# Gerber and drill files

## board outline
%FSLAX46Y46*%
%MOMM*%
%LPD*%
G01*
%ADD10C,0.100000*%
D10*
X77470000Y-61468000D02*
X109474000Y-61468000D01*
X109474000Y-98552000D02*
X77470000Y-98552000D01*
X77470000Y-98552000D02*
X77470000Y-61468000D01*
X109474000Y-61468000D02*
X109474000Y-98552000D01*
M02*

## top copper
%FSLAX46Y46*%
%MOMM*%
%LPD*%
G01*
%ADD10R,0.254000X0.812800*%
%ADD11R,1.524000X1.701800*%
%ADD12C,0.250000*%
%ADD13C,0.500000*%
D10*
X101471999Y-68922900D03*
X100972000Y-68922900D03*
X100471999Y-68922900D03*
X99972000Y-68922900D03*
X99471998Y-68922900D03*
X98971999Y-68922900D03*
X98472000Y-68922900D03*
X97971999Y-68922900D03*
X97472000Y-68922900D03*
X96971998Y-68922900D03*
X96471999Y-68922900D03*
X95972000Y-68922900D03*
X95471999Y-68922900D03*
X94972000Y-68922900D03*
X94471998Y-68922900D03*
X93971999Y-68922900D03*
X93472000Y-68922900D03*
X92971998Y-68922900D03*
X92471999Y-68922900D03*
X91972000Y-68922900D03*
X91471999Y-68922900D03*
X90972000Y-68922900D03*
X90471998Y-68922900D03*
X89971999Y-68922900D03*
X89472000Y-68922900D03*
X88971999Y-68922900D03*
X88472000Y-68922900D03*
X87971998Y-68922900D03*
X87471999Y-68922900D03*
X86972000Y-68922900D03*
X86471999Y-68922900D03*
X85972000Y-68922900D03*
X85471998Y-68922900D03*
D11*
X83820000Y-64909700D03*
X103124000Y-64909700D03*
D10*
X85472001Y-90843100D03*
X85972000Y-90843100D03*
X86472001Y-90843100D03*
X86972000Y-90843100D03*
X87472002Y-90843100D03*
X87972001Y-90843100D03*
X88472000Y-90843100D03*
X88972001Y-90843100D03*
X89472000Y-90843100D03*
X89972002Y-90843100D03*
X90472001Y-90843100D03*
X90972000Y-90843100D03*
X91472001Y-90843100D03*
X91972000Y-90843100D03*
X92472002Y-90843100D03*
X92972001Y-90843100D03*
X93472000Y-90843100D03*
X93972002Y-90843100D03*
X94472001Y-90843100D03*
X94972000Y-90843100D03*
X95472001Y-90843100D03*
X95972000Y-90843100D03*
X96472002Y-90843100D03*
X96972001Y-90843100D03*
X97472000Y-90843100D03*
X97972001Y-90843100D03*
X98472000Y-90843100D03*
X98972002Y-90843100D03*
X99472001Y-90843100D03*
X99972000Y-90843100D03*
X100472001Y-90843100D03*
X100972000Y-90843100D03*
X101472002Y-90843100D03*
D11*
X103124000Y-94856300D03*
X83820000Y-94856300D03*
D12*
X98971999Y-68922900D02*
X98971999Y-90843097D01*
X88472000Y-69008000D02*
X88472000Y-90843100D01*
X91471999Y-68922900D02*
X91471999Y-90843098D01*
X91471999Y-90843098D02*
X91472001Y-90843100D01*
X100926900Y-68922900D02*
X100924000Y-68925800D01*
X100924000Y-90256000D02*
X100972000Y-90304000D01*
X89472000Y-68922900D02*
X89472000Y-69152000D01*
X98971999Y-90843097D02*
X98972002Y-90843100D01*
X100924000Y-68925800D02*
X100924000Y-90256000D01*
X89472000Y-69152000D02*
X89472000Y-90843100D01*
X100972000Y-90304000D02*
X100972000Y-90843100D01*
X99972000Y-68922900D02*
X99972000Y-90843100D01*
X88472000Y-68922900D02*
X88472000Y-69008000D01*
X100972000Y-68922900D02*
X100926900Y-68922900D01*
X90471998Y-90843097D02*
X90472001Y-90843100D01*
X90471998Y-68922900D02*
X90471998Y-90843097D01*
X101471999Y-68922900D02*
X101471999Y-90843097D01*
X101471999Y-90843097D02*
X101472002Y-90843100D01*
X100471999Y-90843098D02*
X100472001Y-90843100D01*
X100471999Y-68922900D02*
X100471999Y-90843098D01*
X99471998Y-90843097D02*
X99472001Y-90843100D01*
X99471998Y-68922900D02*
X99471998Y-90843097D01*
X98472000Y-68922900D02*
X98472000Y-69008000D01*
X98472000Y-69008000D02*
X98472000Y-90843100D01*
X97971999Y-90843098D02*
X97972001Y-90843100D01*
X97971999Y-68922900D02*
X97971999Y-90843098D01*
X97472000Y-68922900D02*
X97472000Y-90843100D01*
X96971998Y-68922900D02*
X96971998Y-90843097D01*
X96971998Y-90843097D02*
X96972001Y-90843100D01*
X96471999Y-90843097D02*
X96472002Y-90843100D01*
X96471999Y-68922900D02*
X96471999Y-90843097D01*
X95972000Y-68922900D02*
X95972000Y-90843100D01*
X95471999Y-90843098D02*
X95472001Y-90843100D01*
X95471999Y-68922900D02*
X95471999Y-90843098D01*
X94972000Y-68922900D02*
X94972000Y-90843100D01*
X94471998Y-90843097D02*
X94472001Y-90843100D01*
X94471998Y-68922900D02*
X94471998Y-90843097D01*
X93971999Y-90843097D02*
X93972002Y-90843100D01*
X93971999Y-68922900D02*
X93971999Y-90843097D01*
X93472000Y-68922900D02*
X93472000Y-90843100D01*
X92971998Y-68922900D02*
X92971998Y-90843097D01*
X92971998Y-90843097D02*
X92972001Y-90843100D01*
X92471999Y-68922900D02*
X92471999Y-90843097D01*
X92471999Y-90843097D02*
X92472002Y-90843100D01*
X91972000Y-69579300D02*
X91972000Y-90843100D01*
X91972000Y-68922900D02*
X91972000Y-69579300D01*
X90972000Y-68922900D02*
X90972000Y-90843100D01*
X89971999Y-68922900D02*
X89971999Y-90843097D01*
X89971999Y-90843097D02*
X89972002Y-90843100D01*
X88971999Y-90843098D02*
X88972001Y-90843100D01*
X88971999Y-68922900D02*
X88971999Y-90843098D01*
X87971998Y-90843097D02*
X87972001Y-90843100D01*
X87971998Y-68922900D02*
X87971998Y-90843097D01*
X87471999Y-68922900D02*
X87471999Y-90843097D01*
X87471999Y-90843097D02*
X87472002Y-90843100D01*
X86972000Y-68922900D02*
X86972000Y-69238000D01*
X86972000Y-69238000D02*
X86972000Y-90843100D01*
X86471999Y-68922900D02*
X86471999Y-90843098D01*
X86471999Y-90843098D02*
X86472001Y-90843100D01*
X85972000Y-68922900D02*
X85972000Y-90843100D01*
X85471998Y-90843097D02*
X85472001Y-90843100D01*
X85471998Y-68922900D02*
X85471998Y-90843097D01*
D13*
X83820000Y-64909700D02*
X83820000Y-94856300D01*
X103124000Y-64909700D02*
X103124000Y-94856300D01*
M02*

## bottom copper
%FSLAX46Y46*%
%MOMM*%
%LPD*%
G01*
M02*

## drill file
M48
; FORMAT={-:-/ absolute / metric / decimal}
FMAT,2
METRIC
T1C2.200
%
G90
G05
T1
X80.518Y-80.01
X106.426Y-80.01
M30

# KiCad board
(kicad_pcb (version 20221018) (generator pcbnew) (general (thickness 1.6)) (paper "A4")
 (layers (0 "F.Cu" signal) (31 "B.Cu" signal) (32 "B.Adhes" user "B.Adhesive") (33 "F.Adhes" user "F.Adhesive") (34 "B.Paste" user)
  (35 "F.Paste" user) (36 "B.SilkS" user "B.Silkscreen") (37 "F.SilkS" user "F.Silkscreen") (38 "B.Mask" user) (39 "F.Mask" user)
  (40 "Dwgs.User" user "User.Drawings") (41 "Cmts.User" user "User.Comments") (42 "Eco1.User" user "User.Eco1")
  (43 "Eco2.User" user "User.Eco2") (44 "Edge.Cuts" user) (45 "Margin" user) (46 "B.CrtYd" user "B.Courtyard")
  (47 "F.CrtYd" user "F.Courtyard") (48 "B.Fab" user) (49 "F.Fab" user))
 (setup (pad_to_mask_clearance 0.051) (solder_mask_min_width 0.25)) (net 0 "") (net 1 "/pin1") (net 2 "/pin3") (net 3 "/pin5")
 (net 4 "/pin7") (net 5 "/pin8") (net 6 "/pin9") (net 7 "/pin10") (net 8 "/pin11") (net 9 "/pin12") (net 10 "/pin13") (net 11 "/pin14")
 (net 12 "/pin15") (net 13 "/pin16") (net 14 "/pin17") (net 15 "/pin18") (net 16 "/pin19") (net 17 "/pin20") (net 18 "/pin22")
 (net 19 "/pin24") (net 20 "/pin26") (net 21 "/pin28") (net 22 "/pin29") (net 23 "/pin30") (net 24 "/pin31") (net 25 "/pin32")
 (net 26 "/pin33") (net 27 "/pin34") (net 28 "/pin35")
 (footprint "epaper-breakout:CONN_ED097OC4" (layer "F.Cu") (at 93.472 71.374)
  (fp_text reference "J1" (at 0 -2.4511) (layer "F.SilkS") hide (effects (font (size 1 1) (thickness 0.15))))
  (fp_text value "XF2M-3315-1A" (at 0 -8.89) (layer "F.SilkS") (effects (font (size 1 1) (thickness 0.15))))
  (pad "1" smd rect (at 7.999999 -2.4511 90) (size 0.8128 0.254) (layers "F.Cu" "F.Paste" "F.Mask") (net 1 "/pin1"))
  (pad "2" smd rect (at 7.5 -2.4511 90) (size 0.8128 0.254) (layers "F.Cu" "F.Paste" "F.Mask"))
  (pad "3" smd rect (at 6.999999 -2.4511 90) (size 0.8128 0.254) (layers "F.Cu" "F.Paste" "F.Mask") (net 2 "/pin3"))
  (pad "4" smd rect (at 6.5 -2.4511 90) (size 0.8128 0.254) (layers "F.Cu" "F.Paste" "F.Mask"))
  (pad "5" smd rect (at 5.999998 -2.4511 90) (size 0.8128 0.254) (layers "F.Cu" "F.Paste" "F.Mask") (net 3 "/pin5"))
  (pad "6" smd rect (at 5.499999 -2.4511 90) (size 0.8128 0.254) (layers "F.Cu" "F.Paste" "F.Mask"))
  (pad "7" smd rect (at 5 -2.4511 90) (size 0.8128 0.254) (layers "F.Cu" "F.Paste" "F.Mask") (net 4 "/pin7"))
  (pad "8" smd rect (at 4.499999 -2.4511 90) (size 0.8128 0.254) (layers "F.Cu" "F.Paste" "F.Mask") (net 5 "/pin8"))
  (pad "9" smd rect (at 4 -2.4511 90) (size 0.8128 0.254) (layers "F.Cu" "F.Paste" "F.Mask") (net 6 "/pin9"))
  (pad "10" smd rect (at 3.499998 -2.4511 90) (size 0.8128 0.254) (layers "F.Cu" "F.Paste" "F.Mask") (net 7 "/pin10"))
  (pad "11" smd rect (at 2.999999 -2.4511 90) (size 0.8128 0.254) (layers "F.Cu" "F.Paste" "F.Mask") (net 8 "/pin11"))
  (pad "12" smd rect (at 2.5 -2.4511 90) (size 0.8128 0.254) (layers "F.Cu" "F.Paste" "F.Mask") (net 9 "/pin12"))
  (pad "13" smd rect (at 1.999999 -2.4511 90) (size 0.8128 0.254) (layers "F.Cu" "F.Paste" "F.Mask") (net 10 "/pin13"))
  (pad "14" smd rect (at 1.5 -2.4511 90) (size 0.8128 0.254) (layers "F.Cu" "F.Paste" "F.Mask") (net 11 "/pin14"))
  (pad "15" smd rect (at 0.999998 -2.4511 90) (size 0.8128 0.254) (layers "F.Cu" "F.Paste" "F.Mask") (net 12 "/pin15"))
  (pad "16" smd rect (at 0.499999 -2.4511 90) (size 0.8128 0.254) (layers "F.Cu" "F.Paste" "F.Mask") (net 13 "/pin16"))
  (pad "17" smd rect (at 0 -2.4511 90) (size 0.8128 0.254) (layers "F.Cu" "F.Paste" "F.Mask") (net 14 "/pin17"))
  (pad "18" smd rect (at -0.500002 -2.4511 90) (size 0.8128 0.254) (layers "F.Cu" "F.Paste" "F.Mask") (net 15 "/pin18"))
  (pad "19" smd rect (at -1.000001 -2.4511 90) (size 0.8128 0.254) (layers "F.Cu" "F.Paste" "F.Mask") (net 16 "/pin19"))
  (pad "20" smd rect (at -1.5 -2.4511 90) (size 0.8128 0.254) (layers "F.Cu" "F.Paste" "F.Mask") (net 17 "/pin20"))
  (pad "21" smd rect (at -2.000001 -2.4511 90) (size 0.8128 0.254) (layers "F.Cu" "F.Paste" "F.Mask"))
  (pad "22" smd rect (at -2.5 -2.4511 90) (size 0.8128 0.254) (layers "F.Cu" "F.Paste" "F.Mask") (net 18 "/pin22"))
  (pad "23" smd rect (at -3.000002 -2.4511 90) (size 0.8128 0.254) (layers "F.Cu" "F.Paste" "F.Mask"))
  (pad "24" smd rect (at -3.500001 -2.4511 90) (size 0.8128 0.254) (layers "F.Cu" "F.Paste" "F.Mask") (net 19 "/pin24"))
  (pad "25" smd rect (at -4 -2.4511 90) (size 0.8128 0.254) (layers "F.Cu" "F.Paste" "F.Mask"))
  (pad "26" smd rect (at -4.500001 -2.4511 90) (size 0.8128 0.254) (layers "F.Cu" "F.Paste" "F.Mask") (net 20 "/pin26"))
  (pad "27" smd rect (at -5 -2.4511 90) (size 0.8128 0.254) (layers "F.Cu" "F.Paste" "F.Mask"))
  (pad "28" smd rect (at -5.500002 -2.4511 90) (size 0.8128 0.254) (layers "F.Cu" "F.Paste" "F.Mask") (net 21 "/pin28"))
  (pad "29" smd rect (at -6.000001 -2.4511 90) (size 0.8128 0.254) (layers "F.Cu" "F.Paste" "F.Mask") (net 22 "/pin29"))
  (pad "30" smd rect (at -6.5 -2.4511 90) (size 0.8128 0.254) (layers "F.Cu" "F.Paste" "F.Mask") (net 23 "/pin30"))
  (pad "31" smd rect (at -7.000001 -2.4511 90) (size 0.8128 0.254) (layers "F.Cu" "F.Paste" "F.Mask") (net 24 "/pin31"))
  (pad "32" smd rect (at -7.5 -2.4511 90) (size 0.8128 0.254) (layers "F.Cu" "F.Paste" "F.Mask") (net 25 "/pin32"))
  (pad "33" smd rect (at -8.000002 -2.4511 90) (size 0.8128 0.254) (layers "F.Cu" "F.Paste" "F.Mask") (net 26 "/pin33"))
  (pad "34" smd rect (at -9.652 -6.4643) (size 1.524 1.7018) (layers "F.Cu" "F.Paste" "F.Mask") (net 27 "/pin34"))
  (pad "35" smd rect (at 9.652 -6.4643) (size 1.524 1.7018) (layers "F.Cu" "F.Paste" "F.Mask") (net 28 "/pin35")))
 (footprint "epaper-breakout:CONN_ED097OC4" (layer "F.Cu") (at 93.472 88.392 180)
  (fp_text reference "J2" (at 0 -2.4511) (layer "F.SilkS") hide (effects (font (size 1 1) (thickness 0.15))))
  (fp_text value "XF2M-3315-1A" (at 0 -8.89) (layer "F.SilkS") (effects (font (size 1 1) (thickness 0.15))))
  (pad "1" smd rect (at 7.999999 -2.4511 270) (size 0.8128 0.254) (layers "F.Cu" "F.Paste" "F.Mask") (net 26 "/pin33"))
  (pad "2" smd rect (at 7.5 -2.4511 270) (size 0.8128 0.254) (layers "F.Cu" "F.Paste" "F.Mask") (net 25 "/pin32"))
  (pad "3" smd rect (at 6.999999 -2.4511 270) (size 0.8128 0.254) (layers "F.Cu" "F.Paste" "F.Mask") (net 24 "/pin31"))
  (pad "4" smd rect (at 6.5 -2.4511 270) (size 0.8128 0.254) (layers "F.Cu" "F.Paste" "F.Mask") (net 23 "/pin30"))
  (pad "5" smd rect (at 5.999998 -2.4511 270) (size 0.8128 0.254) (layers "F.Cu" "F.Paste" "F.Mask") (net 22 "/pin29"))
  (pad "6" smd rect (at 5.499999 -2.4511 270) (size 0.8128 0.254) (layers "F.Cu" "F.Paste" "F.Mask") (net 21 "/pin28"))
  (pad "7" smd rect (at 5 -2.4511 270) (size 0.8128 0.254) (layers "F.Cu" "F.Paste" "F.Mask"))
  (pad "8" smd rect (at 4.499999 -2.4511 270) (size 0.8128 0.254) (layers "F.Cu" "F.Paste" "F.Mask") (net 20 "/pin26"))
  (pad "9" smd rect (at 4 -2.4511 270) (size 0.8128 0.254) (layers "F.Cu" "F.Paste" "F.Mask"))
  (pad "10" smd rect (at 3.499998 -2.4511 270) (size 0.8128 0.254) (layers "F.Cu" "F.Paste" "F.Mask") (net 19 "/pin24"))
  (pad "11" smd rect (at 2.999999 -2.4511 270) (size 0.8128 0.254) (layers "F.Cu" "F.Paste" "F.Mask"))
  (pad "12" smd rect (at 2.5 -2.4511 270) (size 0.8128 0.254) (layers "F.Cu" "F.Paste" "F.Mask") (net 18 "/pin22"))
  (pad "13" smd rect (at 1.999999 -2.4511 270) (size 0.8128 0.254) (layers "F.Cu" "F.Paste" "F.Mask"))
  (pad "14" smd rect (at 1.5 -2.4511 270) (size 0.8128 0.254) (layers "F.Cu" "F.Paste" "F.Mask") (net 17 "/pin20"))
  (pad "15" smd rect (at 0.999998 -2.4511 270) (size 0.8128 0.254) (layers "F.Cu" "F.Paste" "F.Mask") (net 16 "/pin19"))
  (pad "16" smd rect (at 0.499999 -2.4511 270) (size 0.8128 0.254) (layers "F.Cu" "F.Paste" "F.Mask") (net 15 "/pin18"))
  (pad "17" smd rect (at 0 -2.4511 270) (size 0.8128 0.254) (layers "F.Cu" "F.Paste" "F.Mask") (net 14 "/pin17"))
  (pad "18" smd rect (at -0.500002 -2.4511 270) (size 0.8128 0.254) (layers "F.Cu" "F.Paste" "F.Mask") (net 13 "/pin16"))
  (pad "19" smd rect (at -1.000001 -2.4511 270) (size 0.8128 0.254) (layers "F.Cu" "F.Paste" "F.Mask") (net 12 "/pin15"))
  (pad "20" smd rect (at -1.5 -2.4511 270) (size 0.8128 0.254) (layers "F.Cu" "F.Paste" "F.Mask") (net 11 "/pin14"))
  (pad "21" smd rect (at -2.000001 -2.4511 270) (size 0.8128 0.254) (layers "F.Cu" "F.Paste" "F.Mask") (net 10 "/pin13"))
  (pad "22" smd rect (at -2.5 -2.4511 270) (size 0.8128 0.254) (layers "F.Cu" "F.Paste" "F.Mask") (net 9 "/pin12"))
  (pad "23" smd rect (at -3.000002 -2.4511 270) (size 0.8128 0.254) (layers "F.Cu" "F.Paste" "F.Mask") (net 8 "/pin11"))
  (pad "24" smd rect (at -3.500001 -2.4511 270) (size 0.8128 0.254) (layers "F.Cu" "F.Paste" "F.Mask") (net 7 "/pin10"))
  (pad "25" smd rect (at -4 -2.4511 270) (size 0.8128 0.254) (layers "F.Cu" "F.Paste" "F.Mask") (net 6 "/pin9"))
  (pad "26" smd rect (at -4.500001 -2.4511 270) (size 0.8128 0.254) (layers "F.Cu" "F.Paste" "F.Mask") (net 5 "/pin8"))
  (pad "27" smd rect (at -5 -2.4511 270) (size 0.8128 0.254) (layers "F.Cu" "F.Paste" "F.Mask") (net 4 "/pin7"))
  (pad "28" smd rect (at -5.500002 -2.4511 270) (size 0.8128 0.254) (layers "F.Cu" "F.Paste" "F.Mask"))
  (pad "29" smd rect (at -6.000001 -2.4511 270) (size 0.8128 0.254) (layers "F.Cu" "F.Paste" "F.Mask") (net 3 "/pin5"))
  (pad "30" smd rect (at -6.5 -2.4511 270) (size 0.8128 0.254) (layers "F.Cu" "F.Paste" "F.Mask"))
  (pad "31" smd rect (at -7.000001 -2.4511 270) (size 0.8128 0.254) (layers "F.Cu" "F.Paste" "F.Mask") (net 2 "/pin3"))
  (pad "32" smd rect (at -7.5 -2.4511 270) (size 0.8128 0.254) (layers "F.Cu" "F.Paste" "F.Mask"))
  (pad "33" smd rect (at -8.000002 -2.4511 270) (size 0.8128 0.254) (layers "F.Cu" "F.Paste" "F.Mask") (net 1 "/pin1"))
  (pad "34" smd rect (at -9.652 -6.4643 180) (size 1.524 1.7018) (layers "F.Cu" "F.Paste" "F.Mask") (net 28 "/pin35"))
  (pad "35" smd rect (at 9.652 -6.4643 180) (size 1.524 1.7018) (layers "F.Cu" "F.Paste" "F.Mask") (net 27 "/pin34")))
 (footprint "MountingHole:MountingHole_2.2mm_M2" (layer "F.Cu") (at 106.426 80.01)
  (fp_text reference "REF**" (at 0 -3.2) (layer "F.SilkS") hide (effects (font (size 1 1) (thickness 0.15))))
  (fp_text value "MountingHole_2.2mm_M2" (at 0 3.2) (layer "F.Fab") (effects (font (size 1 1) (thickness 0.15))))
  (pad "" np_thru_hole circle (at 0 0) (size 2.2 2.2) (drill 2.2) (layers "*.Cu" "*.Mask")))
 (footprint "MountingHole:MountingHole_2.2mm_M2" (layer "F.Cu") (at 80.518 80.01)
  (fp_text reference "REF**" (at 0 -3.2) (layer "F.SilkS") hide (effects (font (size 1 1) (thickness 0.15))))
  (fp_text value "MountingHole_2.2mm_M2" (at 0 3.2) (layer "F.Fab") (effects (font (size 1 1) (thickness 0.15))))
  (pad "" np_thru_hole circle (at 0 0) (size 2.2 2.2) (drill 2.2) (layers "*.Cu" "*.Mask")))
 (gr_line (start 77.47 61.468) (end 109.474 61.468) (stroke (width 0.1) (type solid)) (layer "Edge.Cuts"))
 (gr_line (start 109.474 98.552) (end 77.47 98.552) (stroke (width 0.1) (type solid)) (layer "Edge.Cuts"))
 (gr_line (start 77.47 98.552) (end 77.47 61.468) (stroke (width 0.1) (type solid)) (layer "Edge.Cuts"))
 (gr_line (start 109.474 61.468) (end 109.474 98.552) (stroke (width 0.1) (type solid)) (layer "Edge.Cuts"))
 (segment (start 98.971999 68.9229) (end 98.971999 90.843097) (width 0.25) (layer "F.Cu") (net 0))
 (segment (start 88.472 69.008) (end 88.472 90.8431) (width 0.25) (layer "F.Cu") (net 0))
 (segment (start 91.471999 68.9229) (end 91.471999 90.843098) (width 0.25) (layer "F.Cu") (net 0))
 (segment (start 91.471999 90.843098) (end 91.472001 90.8431) (width 0.25) (layer "F.Cu") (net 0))
 (segment (start 100.9269 68.9229) (end 100.924 68.9258) (width 0.25) (layer "F.Cu") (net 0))
 (segment (start 100.924 90.256) (end 100.972 90.304) (width 0.25) (layer "F.Cu") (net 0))
 (segment (start 89.472 68.9229) (end 89.472 69.152) (width 0.25) (layer "F.Cu") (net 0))
 (segment (start 98.971999 90.843097) (end 98.972002 90.8431) (width 0.25) (layer "F.Cu") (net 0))
 (segment (start 100.924 68.9258) (end 100.924 90.256) (width 0.25) (layer "F.Cu") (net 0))
 (segment (start 89.472 69.152) (end 89.472 90.8431) (width 0.25) (layer "F.Cu") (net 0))
 (segment (start 100.972 90.304) (end 100.972 90.8431) (width 0.25) (layer "F.Cu") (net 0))
 (segment (start 99.972 68.9229) (end 99.972 90.8431) (width 0.25) (layer "F.Cu") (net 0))
 (segment (start 88.472 68.9229) (end 88.472 69.008) (width 0.25) (layer "F.Cu") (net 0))
 (segment (start 100.972 68.9229) (end 100.9269 68.9229) (width 0.25) (layer "F.Cu") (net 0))
 (segment (start 90.471998 90.843097) (end 90.472001 90.8431) (width 0.25) (layer "F.Cu") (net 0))
 (segment (start 90.471998 68.9229) (end 90.471998 90.843097) (width 0.25) (layer "F.Cu") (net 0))
 (segment (start 101.471999 68.9229) (end 101.471999 90.843097) (width 0.25) (layer "F.Cu") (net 1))
 (segment (start 101.471999 90.843097) (end 101.472002 90.8431) (width 0.25) (layer "F.Cu") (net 1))
 (segment (start 100.471999 90.843098) (end 100.472001 90.8431) (width 0.25) (layer "F.Cu") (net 2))
 (segment (start 100.471999 68.9229) (end 100.471999 90.843098) (width 0.25) (layer "F.Cu") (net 2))
 (segment (start 99.471998 90.843097) (end 99.472001 90.8431) (width 0.25) (layer "F.Cu") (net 3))
 (segment (start 99.471998 68.9229) (end 99.471998 90.843097) (width 0.25) (layer "F.Cu") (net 3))
 (segment (start 98.472 68.9229) (end 98.472 69.008) (width 0.25) (layer "F.Cu") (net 4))
 (segment (start 98.472 69.008) (end 98.472 90.8431) (width 0.25) (layer "F.Cu") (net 4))
 (segment (start 97.971999 90.843098) (end 97.972001 90.8431) (width 0.25) (layer "F.Cu") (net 5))
 (segment (start 97.971999 68.9229) (end 97.971999 90.843098) (width 0.25) (layer "F.Cu") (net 5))
 (segment (start 97.472 68.9229) (end 97.472 90.8431) (width 0.25) (layer "F.Cu") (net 6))
 (segment (start 96.971998 68.9229) (end 96.971998 90.843097) (width 0.25) (layer "F.Cu") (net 7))
 (segment (start 96.971998 90.843097) (end 96.972001 90.8431) (width 0.25) (layer "F.Cu") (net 7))
 (segment (start 96.471999 90.843097) (end 96.472002 90.8431) (width 0.25) (layer "F.Cu") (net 8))
 (segment (start 96.471999 68.9229) (end 96.471999 90.843097) (width 0.25) (layer "F.Cu") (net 8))
 (segment (start 95.972 68.9229) (end 95.972 90.8431) (width 0.25) (layer "F.Cu") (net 9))
 (segment (start 95.471999 90.843098) (end 95.472001 90.8431) (width 0.25) (layer "F.Cu") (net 10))
 (segment (start 95.471999 68.9229) (end 95.471999 90.843098) (width 0.25) (layer "F.Cu") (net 10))
 (segment (start 94.972 68.9229) (end 94.972 90.8431) (width 0.25) (layer "F.Cu") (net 11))
 (segment (start 94.471998 90.843097) (end 94.472001 90.8431) (width 0.25) (layer "F.Cu") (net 12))
 (segment (start 94.471998 68.9229) (end 94.471998 90.843097) (width 0.25) (layer "F.Cu") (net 12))
 (segment (start 93.971999 90.843097) (end 93.972002 90.8431) (width 0.25) (layer "F.Cu") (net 13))
 (segment (start 93.971999 68.9229) (end 93.971999 90.843097) (width 0.25) (layer "F.Cu") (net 13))
 (segment (start 93.472 68.9229) (end 93.472 90.8431) (width 0.25) (layer "F.Cu") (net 14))
 (segment (start 92.971998 68.9229) (end 92.971998 90.843097) (width 0.25) (layer "F.Cu") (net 15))
 (segment (start 92.971998 90.843097) (end 92.972001 90.8431) (width 0.25) (layer "F.Cu") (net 15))
 (segment (start 92.471999 68.9229) (end 92.471999 90.843097) (width 0.25) (layer "F.Cu") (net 16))
 (segment (start 92.471999 90.843097) (end 92.472002 90.8431) (width 0.25) (layer "F.Cu") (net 16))
 (segment (start 91.972 69.5793) (end 91.972 90.8431) (width 0.25) (layer "F.Cu") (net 17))
 (segment (start 91.972 68.9229) (end 91.972 69.5793) (width 0.25) (layer "F.Cu") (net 17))
 (segment (start 90.972 68.9229) (end 90.972 90.8431) (width 0.25) (layer "F.Cu") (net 18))
 (segment (start 89.971999 68.9229) (end 89.971999 90.843097) (width 0.25) (layer "F.Cu") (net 19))
 (segment (start 89.971999 90.843097) (end 89.972002 90.8431) (width 0.25) (layer "F.Cu") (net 19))
 (segment (start 88.971999 90.843098) (end 88.972001 90.8431) (width 0.25) (layer "F.Cu") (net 20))
 (segment (start 88.971999 68.9229) (end 88.971999 90.843098) (width 0.25) (layer "F.Cu") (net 20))
 (segment (start 87.971998 90.843097) (end 87.972001 90.8431) (width 0.25) (layer "F.Cu") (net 21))
 (segment (start 87.971998 68.9229) (end 87.971998 90.843097) (width 0.25) (layer "F.Cu") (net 21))
 (segment (start 87.471999 68.9229) (end 87.471999 90.843097) (width 0.25) (layer "F.Cu") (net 22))
 (segment (start 87.471999 90.843097) (end 87.472002 90.8431) (width 0.25) (layer "F.Cu") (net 22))
 (segment (start 86.972 68.9229) (end 86.972 69.238) (width 0.25) (layer "F.Cu") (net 23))
 (segment (start 86.972 69.238) (end 86.972 90.8431) (width 0.25) (layer "F.Cu") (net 23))
 (segment (start 86.471999 68.9229) (end 86.471999 90.843098) (width 0.25) (layer "F.Cu") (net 24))
 (segment (start 86.471999 90.843098) (end 86.472001 90.8431) (width 0.25) (layer "F.Cu") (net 24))
 (segment (start 85.972 68.9229) (end 85.972 90.8431) (width 0.25) (layer "F.Cu") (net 25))
 (segment (start 85.471998 90.843097) (end 85.472001 90.8431) (width 0.25) (layer "F.Cu") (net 26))
 (segment (start 85.471998 68.9229) (end 85.471998 90.843097) (width 0.25) (layer "F.Cu") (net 26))
 (segment (start 83.82 64.9097) (end 83.82 94.8563) (width 0.5) (layer "F.Cu") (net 27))
 (segment (start 103.124 64.9097) (end 103.124 94.8563) (width 0.5) (layer "F.Cu") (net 28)))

